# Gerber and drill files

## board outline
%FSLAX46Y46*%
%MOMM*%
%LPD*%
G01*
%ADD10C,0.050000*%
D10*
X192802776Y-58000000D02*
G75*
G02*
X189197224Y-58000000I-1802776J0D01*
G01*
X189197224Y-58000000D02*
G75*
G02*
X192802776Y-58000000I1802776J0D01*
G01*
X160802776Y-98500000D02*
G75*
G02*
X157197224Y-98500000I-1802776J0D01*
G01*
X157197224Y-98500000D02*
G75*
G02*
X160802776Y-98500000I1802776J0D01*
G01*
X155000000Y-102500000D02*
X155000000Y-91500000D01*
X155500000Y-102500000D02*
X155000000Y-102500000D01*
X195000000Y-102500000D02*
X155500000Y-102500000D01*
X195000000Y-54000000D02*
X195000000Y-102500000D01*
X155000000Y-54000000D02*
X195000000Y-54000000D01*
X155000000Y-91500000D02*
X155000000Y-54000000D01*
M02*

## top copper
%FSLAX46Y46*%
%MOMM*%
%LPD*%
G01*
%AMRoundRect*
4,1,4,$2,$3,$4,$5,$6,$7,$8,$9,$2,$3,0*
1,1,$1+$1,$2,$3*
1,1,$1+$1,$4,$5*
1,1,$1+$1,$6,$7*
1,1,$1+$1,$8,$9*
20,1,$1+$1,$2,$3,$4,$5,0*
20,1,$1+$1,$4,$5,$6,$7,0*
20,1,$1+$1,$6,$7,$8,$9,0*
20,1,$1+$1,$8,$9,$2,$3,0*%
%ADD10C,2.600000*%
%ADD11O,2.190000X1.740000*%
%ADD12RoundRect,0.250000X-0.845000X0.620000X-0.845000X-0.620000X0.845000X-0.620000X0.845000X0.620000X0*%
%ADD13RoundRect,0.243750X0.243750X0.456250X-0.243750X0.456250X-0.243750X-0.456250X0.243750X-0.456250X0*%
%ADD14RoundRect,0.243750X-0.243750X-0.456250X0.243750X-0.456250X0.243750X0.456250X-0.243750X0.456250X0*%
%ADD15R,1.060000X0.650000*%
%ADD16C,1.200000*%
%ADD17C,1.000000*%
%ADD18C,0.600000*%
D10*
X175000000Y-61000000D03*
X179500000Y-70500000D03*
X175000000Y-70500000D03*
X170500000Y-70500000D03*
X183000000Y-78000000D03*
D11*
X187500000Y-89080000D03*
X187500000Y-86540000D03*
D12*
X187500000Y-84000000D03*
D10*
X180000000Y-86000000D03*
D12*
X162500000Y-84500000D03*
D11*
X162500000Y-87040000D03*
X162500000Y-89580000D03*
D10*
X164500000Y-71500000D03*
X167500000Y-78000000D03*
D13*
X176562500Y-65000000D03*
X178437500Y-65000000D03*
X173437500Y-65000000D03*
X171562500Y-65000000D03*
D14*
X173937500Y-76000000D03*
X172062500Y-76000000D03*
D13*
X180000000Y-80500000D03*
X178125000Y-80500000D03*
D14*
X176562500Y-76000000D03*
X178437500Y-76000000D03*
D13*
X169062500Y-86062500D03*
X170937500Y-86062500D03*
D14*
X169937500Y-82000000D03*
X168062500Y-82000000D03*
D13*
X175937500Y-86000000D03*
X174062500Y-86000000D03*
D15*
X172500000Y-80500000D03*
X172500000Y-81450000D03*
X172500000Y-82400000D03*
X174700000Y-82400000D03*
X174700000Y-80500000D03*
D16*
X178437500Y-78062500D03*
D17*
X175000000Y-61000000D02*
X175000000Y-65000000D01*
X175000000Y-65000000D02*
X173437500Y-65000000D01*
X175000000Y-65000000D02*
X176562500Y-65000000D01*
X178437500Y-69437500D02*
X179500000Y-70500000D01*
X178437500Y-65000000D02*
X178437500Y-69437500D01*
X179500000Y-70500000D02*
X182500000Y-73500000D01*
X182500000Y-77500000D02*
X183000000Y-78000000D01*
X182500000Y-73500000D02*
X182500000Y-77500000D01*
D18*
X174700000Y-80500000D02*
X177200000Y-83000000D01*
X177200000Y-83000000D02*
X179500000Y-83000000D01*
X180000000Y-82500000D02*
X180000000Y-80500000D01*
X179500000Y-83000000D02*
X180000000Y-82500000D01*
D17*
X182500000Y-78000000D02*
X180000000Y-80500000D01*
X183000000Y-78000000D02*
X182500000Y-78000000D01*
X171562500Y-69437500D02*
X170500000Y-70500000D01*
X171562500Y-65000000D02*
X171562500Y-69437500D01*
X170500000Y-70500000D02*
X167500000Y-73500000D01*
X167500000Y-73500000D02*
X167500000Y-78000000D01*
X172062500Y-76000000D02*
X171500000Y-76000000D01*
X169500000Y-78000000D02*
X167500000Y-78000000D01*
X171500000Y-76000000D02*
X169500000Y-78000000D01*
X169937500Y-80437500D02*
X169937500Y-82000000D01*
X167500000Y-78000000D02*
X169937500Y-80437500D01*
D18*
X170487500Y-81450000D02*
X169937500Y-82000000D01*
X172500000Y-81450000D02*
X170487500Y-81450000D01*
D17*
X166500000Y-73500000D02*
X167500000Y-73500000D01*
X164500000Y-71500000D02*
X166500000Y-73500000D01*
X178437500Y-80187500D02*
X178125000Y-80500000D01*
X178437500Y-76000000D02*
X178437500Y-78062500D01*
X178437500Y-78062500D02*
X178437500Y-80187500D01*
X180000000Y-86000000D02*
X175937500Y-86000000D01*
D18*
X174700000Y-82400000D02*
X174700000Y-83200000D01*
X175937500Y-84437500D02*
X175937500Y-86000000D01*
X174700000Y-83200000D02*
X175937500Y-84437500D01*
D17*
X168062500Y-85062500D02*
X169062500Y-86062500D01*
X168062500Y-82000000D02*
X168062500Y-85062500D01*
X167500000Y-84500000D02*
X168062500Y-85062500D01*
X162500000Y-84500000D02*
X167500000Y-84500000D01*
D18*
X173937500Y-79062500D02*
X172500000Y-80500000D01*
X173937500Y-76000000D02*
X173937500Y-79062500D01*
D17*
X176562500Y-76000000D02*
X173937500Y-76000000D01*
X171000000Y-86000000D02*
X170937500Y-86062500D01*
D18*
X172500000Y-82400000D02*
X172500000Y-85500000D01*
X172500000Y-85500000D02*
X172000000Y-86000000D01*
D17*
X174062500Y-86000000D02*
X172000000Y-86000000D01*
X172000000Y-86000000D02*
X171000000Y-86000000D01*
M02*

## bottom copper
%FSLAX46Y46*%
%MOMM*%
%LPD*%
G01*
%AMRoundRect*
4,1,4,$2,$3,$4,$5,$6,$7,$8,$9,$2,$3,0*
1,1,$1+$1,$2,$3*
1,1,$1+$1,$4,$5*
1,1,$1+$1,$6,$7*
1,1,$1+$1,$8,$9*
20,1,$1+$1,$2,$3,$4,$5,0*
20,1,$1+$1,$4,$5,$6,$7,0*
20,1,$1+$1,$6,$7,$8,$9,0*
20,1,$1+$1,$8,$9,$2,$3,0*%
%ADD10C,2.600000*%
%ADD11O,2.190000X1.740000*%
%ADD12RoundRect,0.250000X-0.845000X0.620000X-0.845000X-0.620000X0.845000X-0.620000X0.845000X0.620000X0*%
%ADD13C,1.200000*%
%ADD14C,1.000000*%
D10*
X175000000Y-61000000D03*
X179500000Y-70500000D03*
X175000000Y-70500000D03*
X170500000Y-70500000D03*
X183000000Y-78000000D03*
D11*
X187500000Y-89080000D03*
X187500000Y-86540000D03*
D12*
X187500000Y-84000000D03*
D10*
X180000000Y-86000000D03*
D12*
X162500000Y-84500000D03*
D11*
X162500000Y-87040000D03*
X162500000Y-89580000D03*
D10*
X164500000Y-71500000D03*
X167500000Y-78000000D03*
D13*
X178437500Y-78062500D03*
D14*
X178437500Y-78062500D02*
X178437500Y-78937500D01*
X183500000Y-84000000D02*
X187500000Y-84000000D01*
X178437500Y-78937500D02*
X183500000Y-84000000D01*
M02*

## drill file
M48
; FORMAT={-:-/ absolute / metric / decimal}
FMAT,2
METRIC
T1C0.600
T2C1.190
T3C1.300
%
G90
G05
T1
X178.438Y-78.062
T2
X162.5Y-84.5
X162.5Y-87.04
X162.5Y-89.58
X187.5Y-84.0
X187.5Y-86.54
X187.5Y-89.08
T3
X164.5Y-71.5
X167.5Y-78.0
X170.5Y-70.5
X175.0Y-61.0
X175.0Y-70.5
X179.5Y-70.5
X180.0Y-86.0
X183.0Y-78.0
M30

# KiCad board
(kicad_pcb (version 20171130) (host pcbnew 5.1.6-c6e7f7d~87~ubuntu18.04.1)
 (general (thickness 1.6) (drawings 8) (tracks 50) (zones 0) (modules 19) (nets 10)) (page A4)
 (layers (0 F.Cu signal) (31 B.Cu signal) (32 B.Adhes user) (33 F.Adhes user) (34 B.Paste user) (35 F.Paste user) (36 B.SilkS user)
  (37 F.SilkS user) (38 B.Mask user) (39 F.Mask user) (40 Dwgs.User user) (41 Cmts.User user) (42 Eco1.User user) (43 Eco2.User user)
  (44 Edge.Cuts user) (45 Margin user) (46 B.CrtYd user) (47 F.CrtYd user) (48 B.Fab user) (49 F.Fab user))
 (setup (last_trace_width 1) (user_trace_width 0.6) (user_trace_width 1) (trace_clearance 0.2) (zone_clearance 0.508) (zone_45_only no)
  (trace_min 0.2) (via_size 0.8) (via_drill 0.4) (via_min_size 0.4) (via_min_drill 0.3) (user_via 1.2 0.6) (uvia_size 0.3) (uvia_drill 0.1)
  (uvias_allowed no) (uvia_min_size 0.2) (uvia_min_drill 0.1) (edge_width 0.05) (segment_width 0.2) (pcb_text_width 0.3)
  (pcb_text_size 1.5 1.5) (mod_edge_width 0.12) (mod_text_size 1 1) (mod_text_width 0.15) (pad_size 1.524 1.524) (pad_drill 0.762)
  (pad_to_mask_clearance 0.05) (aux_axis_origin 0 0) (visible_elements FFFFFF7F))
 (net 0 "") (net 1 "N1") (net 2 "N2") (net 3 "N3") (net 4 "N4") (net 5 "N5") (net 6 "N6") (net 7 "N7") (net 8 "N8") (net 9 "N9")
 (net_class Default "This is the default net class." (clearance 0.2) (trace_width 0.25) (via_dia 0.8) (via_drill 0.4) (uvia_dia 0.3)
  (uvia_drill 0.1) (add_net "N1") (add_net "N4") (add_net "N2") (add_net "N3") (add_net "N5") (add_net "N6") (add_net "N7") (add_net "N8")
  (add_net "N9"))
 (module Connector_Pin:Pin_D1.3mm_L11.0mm (layer F.Cu) (at 175 61)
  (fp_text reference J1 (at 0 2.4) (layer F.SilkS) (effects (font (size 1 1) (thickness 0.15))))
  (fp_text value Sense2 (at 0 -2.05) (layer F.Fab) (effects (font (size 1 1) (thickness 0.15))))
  (pad 1 thru_hole circle (at 0 0) (size 2.6 2.6) (drill 1.3) (layers *.Cu *.Mask) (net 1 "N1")))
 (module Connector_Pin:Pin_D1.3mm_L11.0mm (layer F.Cu) (at 179.5 70.5)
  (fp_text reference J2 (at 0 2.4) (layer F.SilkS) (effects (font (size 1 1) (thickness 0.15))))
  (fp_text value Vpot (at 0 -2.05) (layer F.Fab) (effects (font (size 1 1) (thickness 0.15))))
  (pad 1 thru_hole circle (at 0 0) (size 2.6 2.6) (drill 1.3) (layers *.Cu *.Mask) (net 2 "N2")))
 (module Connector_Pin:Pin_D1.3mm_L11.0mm (layer F.Cu) (at 175 70.5)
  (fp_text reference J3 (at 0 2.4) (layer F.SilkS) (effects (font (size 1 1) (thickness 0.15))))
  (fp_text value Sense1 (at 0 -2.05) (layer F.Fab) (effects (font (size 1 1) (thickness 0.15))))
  (pad 1 thru_hole circle (at 0 0) (size 2.6 2.6) (drill 1.3) (layers *.Cu *.Mask) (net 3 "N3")))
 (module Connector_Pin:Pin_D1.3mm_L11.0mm (layer F.Cu) (at 170.5 70.5)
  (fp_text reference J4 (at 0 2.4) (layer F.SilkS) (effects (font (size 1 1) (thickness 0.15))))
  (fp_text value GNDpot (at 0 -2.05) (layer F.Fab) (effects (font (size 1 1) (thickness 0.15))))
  (pad 1 thru_hole circle (at 0 0) (size 2.6 2.6) (drill 1.3) (layers *.Cu *.Mask) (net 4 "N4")))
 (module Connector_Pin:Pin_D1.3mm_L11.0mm (layer F.Cu) (at 183 78)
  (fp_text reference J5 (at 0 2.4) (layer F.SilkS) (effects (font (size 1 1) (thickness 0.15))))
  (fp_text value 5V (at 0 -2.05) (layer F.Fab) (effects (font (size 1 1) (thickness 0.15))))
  (pad 1 thru_hole circle (at 0 0) (size 2.6 2.6) (drill 1.3) (layers *.Cu *.Mask) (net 2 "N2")))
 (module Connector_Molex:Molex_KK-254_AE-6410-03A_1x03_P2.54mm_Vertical (layer F.Cu) (at 187.5 84 270)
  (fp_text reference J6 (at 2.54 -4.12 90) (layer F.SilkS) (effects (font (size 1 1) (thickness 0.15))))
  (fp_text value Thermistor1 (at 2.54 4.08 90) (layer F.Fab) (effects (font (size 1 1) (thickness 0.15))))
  (pad 3 thru_hole oval (at 5.08 0 270) (size 1.74 2.19) (drill 1.19) (layers *.Cu *.Mask))
  (pad 2 thru_hole oval (at 2.54 0 270) (size 1.74 2.19) (drill 1.19) (layers *.Cu *.Mask))
  (pad 1 thru_hole roundrect (at 0 0 270) (size 1.74 2.19) (drill 1.19) (layers *.Cu *.Mask) (roundrect_rratio 0.143678) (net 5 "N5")))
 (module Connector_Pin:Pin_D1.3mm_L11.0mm (layer F.Cu) (at 180 86)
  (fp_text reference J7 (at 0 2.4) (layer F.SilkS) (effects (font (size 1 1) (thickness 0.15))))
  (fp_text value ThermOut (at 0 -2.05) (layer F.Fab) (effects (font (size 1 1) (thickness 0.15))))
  (pad 1 thru_hole circle (at 0 0) (size 2.6 2.6) (drill 1.3) (layers *.Cu *.Mask) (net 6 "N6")))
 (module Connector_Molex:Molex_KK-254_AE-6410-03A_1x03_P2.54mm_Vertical (layer F.Cu) (at 162.5 84.5 270)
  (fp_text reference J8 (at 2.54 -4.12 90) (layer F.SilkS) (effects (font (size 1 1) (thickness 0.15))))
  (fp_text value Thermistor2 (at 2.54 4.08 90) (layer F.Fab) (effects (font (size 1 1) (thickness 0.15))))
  (pad 1 thru_hole roundrect (at 0 0 270) (size 1.74 2.19) (drill 1.19) (layers *.Cu *.Mask) (roundrect_rratio 0.143678) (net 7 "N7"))
  (pad 2 thru_hole oval (at 2.54 0 270) (size 1.74 2.19) (drill 1.19) (layers *.Cu *.Mask))
  (pad 3 thru_hole oval (at 5.08 0 270) (size 1.74 2.19) (drill 1.19) (layers *.Cu *.Mask)))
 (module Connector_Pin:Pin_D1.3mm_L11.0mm (layer F.Cu) (at 164.5 71.5)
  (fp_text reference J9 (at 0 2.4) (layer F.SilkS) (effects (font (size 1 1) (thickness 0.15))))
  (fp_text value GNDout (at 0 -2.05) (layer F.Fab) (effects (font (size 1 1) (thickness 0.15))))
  (pad 1 thru_hole circle (at 0 0) (size 2.6 2.6) (drill 1.3) (layers *.Cu *.Mask) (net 4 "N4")))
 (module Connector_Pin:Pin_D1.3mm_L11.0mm (layer F.Cu) (at 167.5 78)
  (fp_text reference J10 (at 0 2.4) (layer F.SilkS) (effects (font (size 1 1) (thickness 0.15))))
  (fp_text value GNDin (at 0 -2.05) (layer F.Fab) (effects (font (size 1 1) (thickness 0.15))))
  (pad 1 thru_hole circle (at 0 0) (size 2.6 2.6) (drill 1.3) (layers *.Cu *.Mask) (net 4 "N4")))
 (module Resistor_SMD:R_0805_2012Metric (layer F.Cu) (at 177.5 65 180)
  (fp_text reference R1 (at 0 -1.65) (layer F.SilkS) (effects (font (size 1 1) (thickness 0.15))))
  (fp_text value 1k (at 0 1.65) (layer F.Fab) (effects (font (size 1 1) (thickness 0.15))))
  (pad 2 smd roundrect (at 0.9375 0 180) (size 0.975 1.4) (layers F.Cu F.Paste F.Mask) (roundrect_rratio 0.25) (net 1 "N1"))
  (pad 1 smd roundrect (at -0.9375 0 180) (size 0.975 1.4) (layers F.Cu F.Paste F.Mask) (roundrect_rratio 0.25) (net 2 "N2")))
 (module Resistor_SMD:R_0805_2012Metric (layer F.Cu) (at 172.5 65 180)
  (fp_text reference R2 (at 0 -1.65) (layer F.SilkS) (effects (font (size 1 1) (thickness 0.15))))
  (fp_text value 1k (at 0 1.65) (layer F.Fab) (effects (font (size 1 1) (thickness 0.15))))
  (pad 1 smd roundrect (at -0.9375 0 180) (size 0.975 1.4) (layers F.Cu F.Paste F.Mask) (roundrect_rratio 0.25) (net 1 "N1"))
  (pad 2 smd roundrect (at 0.9375 0 180) (size 0.975 1.4) (layers F.Cu F.Paste F.Mask) (roundrect_rratio 0.25) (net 4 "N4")))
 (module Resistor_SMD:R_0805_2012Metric (layer F.Cu) (at 173 76)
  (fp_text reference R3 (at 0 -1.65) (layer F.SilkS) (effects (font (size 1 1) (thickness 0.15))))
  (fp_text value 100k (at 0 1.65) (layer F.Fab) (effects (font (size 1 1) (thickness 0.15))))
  (pad 2 smd roundrect (at 0.9375 0) (size 0.975 1.4) (layers F.Cu F.Paste F.Mask) (roundrect_rratio 0.25) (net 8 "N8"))
  (pad 1 smd roundrect (at -0.9375 0) (size 0.975 1.4) (layers F.Cu F.Paste F.Mask) (roundrect_rratio 0.25) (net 4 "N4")))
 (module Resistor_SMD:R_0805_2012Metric (layer F.Cu) (at 179.0625 80.5 180)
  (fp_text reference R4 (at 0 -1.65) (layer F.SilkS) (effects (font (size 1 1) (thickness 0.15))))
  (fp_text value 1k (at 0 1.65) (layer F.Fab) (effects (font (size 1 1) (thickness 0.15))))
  (pad 1 smd roundrect (at -0.9375 0 180) (size 0.975 1.4) (layers F.Cu F.Paste F.Mask) (roundrect_rratio 0.25) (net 2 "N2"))
  (pad 2 smd roundrect (at 0.9375 0 180) (size 0.975 1.4) (layers F.Cu F.Paste F.Mask) (roundrect_rratio 0.25) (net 5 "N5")))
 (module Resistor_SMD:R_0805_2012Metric (layer F.Cu) (at 177.5 76)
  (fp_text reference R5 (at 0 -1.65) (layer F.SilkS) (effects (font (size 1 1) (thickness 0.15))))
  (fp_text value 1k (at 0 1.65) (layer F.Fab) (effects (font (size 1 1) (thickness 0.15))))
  (pad 1 smd roundrect (at -0.9375 0) (size 0.975 1.4) (layers F.Cu F.Paste F.Mask) (roundrect_rratio 0.25) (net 8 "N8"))
  (pad 2 smd roundrect (at 0.9375 0) (size 0.975 1.4) (layers F.Cu F.Paste F.Mask) (roundrect_rratio 0.25) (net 5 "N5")))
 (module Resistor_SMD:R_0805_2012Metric (layer F.Cu) (at 170 86.0625 180)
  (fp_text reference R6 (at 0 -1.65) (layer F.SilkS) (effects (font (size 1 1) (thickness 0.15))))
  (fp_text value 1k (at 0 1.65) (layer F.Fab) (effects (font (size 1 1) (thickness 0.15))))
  (pad 2 smd roundrect (at 0.9375 0 180) (size 0.975 1.4) (layers F.Cu F.Paste F.Mask) (roundrect_rratio 0.25) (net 7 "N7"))
  (pad 1 smd roundrect (at -0.9375 0 180) (size 0.975 1.4) (layers F.Cu F.Paste F.Mask) (roundrect_rratio 0.25) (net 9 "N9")))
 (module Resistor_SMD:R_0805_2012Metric (layer F.Cu) (at 169 82)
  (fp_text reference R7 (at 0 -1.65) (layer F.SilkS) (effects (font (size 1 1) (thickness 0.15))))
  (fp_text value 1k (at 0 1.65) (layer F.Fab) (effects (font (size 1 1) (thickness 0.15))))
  (pad 2 smd roundrect (at 0.9375 0) (size 0.975 1.4) (layers F.Cu F.Paste F.Mask) (roundrect_rratio 0.25) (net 4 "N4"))
  (pad 1 smd roundrect (at -0.9375 0) (size 0.975 1.4) (layers F.Cu F.Paste F.Mask) (roundrect_rratio 0.25) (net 7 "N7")))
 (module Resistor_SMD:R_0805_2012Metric (layer F.Cu) (at 175 86 180)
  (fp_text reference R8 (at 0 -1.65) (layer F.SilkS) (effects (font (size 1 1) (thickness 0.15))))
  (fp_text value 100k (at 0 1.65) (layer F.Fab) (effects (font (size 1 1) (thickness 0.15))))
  (pad 1 smd roundrect (at -0.9375 0 180) (size 0.975 1.4) (layers F.Cu F.Paste F.Mask) (roundrect_rratio 0.25) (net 6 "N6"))
  (pad 2 smd roundrect (at 0.9375 0 180) (size 0.975 1.4) (layers F.Cu F.Paste F.Mask) (roundrect_rratio 0.25) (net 9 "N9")))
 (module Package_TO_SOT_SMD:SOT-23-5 (layer F.Cu) (at 173.6 81.45)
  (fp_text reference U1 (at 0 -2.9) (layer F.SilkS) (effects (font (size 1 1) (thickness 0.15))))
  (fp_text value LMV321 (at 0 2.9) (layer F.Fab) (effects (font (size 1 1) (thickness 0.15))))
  (pad 1 smd rect (at -1.1 -0.95) (size 1.06 0.65) (layers F.Cu F.Paste F.Mask) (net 8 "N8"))
  (pad 2 smd rect (at -1.1 0) (size 1.06 0.65) (layers F.Cu F.Paste F.Mask) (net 4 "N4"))
  (pad 3 smd rect (at -1.1 0.95) (size 1.06 0.65) (layers F.Cu F.Paste F.Mask) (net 9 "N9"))
  (pad 4 smd rect (at 1.1 0.95) (size 1.06 0.65) (layers F.Cu F.Paste F.Mask) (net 6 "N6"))
  (pad 5 smd rect (at 1.1 -0.95) (size 1.06 0.65) (layers F.Cu F.Paste F.Mask) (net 2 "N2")))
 (gr_circle (center 191 58) (end 192 59.5) (layer Edge.Cuts) (width 0.05))
 (gr_circle (center 159 98.5) (end 160.5 99.5) (layer Edge.Cuts) (width 0.05))
 (gr_line (start 155 102.5) (end 155 91.5) (layer Edge.Cuts) (width 0.05))
 (gr_line (start 155.5 102.5) (end 155 102.5) (layer Edge.Cuts) (width 0.05))
 (gr_line (start 195 102.5) (end 155.5 102.5) (layer Edge.Cuts) (width 0.05))
 (gr_line (start 195 54) (end 195 102.5) (layer Edge.Cuts) (width 0.05))
 (gr_line (start 155 54) (end 195 54) (layer Edge.Cuts) (width 0.05))
 (gr_line (start 155 91.5) (end 155 54) (layer Edge.Cuts) (width 0.05))
 (segment (start 175 61) (end 175 65) (width 1) (layer F.Cu) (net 1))
 (segment (start 175 65) (end 173.4375 65) (width 1) (layer F.Cu) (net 1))
 (segment (start 175 65) (end 176.5625 65) (width 1) (layer F.Cu) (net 1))
 (segment (start 178.4375 69.4375) (end 179.5 70.5) (width 1) (layer F.Cu) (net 2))
 (segment (start 178.4375 65) (end 178.4375 69.4375) (width 1) (layer F.Cu) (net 2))
 (segment (start 179.5 70.5) (end 182.5 73.5) (width 1) (layer F.Cu) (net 2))
 (segment (start 182.5 77.5) (end 183 78) (width 1) (layer F.Cu) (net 2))
 (segment (start 182.5 73.5) (end 182.5 77.5) (width 1) (layer F.Cu) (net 2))
 (segment (start 174.7 80.5) (end 177.2 83) (width 0.6) (layer F.Cu) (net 2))
 (segment (start 177.2 83) (end 179.5 83) (width 0.6) (layer F.Cu) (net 2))
 (segment (start 180 82.5) (end 180 80.5) (width 0.6) (layer F.Cu) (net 2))
 (segment (start 179.5 83) (end 180 82.5) (width 0.6) (layer F.Cu) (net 2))
 (segment (start 182.5 78) (end 180 80.5) (width 1) (layer F.Cu) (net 2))
 (segment (start 183 78) (end 182.5 78) (width 1) (layer F.Cu) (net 2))
 (segment (start 171.5625 69.4375) (end 170.5 70.5) (width 1) (layer F.Cu) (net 4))
 (segment (start 171.5625 65) (end 171.5625 69.4375) (width 1) (layer F.Cu) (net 4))
 (segment (start 170.5 70.5) (end 167.5 73.5) (width 1) (layer F.Cu) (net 4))
 (segment (start 167.5 73.5) (end 167.5 78) (width 1) (layer F.Cu) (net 4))
 (segment (start 172.0625 76) (end 171.5 76) (width 1) (layer F.Cu) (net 4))
 (segment (start 169.5 78) (end 167.5 78) (width 1) (layer F.Cu) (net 4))
 (segment (start 171.5 76) (end 169.5 78) (width 1) (layer F.Cu) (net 4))
 (segment (start 169.9375 80.4375) (end 169.9375 82) (width 1) (layer F.Cu) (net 4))
 (segment (start 167.5 78) (end 169.9375 80.4375) (width 1) (layer F.Cu) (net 4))
 (segment (start 170.4875 81.45) (end 169.9375 82) (width 0.6) (layer F.Cu) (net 4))
 (segment (start 172.5 81.45) (end 170.4875 81.45) (width 0.6) (layer F.Cu) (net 4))
 (segment (start 166.5 73.5) (end 167.5 73.5) (width 1) (layer F.Cu) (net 4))
 (segment (start 164.5 71.5) (end 166.5 73.5) (width 1) (layer F.Cu) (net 4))
 (segment (start 178.4375 80.1875) (end 178.125 80.5) (width 1) (layer F.Cu) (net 5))
 (segment (start 178.4375 76) (end 178.4375 78.0625) (width 1) (layer F.Cu) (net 5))
 (segment (start 178.4375 78.0625) (end 178.4375 80.1875) (width 1) (layer F.Cu) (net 5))
 (via (at 178.4375 78.0625) (size 1.2) (drill 0.6) (layers F.Cu B.Cu) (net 5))
 (segment (start 178.4375 78.0625) (end 178.4375 78.9375) (width 1) (layer B.Cu) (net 5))
 (segment (start 183.5 84) (end 187.5 84) (width 1) (layer B.Cu) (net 5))
 (segment (start 178.4375 78.9375) (end 183.5 84) (width 1) (layer B.Cu) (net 5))
 (segment (start 180 86) (end 175.9375 86) (width 1) (layer F.Cu) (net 6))
 (segment (start 174.7 82.4) (end 174.7 83.2) (width 0.6) (layer F.Cu) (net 6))
 (segment (start 175.9375 84.4375) (end 175.9375 86) (width 0.6) (layer F.Cu) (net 6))
 (segment (start 174.7 83.2) (end 175.9375 84.4375) (width 0.6) (layer F.Cu) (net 6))
 (segment (start 168.0625 85.0625) (end 169.0625 86.0625) (width 1) (layer F.Cu) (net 7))
 (segment (start 168.0625 82) (end 168.0625 85.0625) (width 1) (layer F.Cu) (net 7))
 (segment (start 167.5 84.5) (end 168.0625 85.0625) (width 1) (layer F.Cu) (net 7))
 (segment (start 162.5 84.5) (end 167.5 84.5) (width 1) (layer F.Cu) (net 7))
 (segment (start 173.9375 79.0625) (end 172.5 80.5) (width 0.6) (layer F.Cu) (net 8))
 (segment (start 173.9375 76) (end 173.9375 79.0625) (width 0.6) (layer F.Cu) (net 8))
 (segment (start 176.5625 76) (end 173.9375 76) (width 1) (layer F.Cu) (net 8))
 (segment (start 171 86) (end 170.9375 86.0625) (width 1) (layer F.Cu) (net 9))
 (segment (start 172.5 82.4) (end 172.5 85.5) (width 0.6) (layer F.Cu) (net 9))
 (segment (start 172.5 85.5) (end 172 86) (width 0.6) (layer F.Cu) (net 9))
 (segment (start 174.0625 86) (end 172 86) (width 1) (layer F.Cu) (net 9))
 (segment (start 172 86) (end 171 86) (width 1) (layer F.Cu) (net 9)))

